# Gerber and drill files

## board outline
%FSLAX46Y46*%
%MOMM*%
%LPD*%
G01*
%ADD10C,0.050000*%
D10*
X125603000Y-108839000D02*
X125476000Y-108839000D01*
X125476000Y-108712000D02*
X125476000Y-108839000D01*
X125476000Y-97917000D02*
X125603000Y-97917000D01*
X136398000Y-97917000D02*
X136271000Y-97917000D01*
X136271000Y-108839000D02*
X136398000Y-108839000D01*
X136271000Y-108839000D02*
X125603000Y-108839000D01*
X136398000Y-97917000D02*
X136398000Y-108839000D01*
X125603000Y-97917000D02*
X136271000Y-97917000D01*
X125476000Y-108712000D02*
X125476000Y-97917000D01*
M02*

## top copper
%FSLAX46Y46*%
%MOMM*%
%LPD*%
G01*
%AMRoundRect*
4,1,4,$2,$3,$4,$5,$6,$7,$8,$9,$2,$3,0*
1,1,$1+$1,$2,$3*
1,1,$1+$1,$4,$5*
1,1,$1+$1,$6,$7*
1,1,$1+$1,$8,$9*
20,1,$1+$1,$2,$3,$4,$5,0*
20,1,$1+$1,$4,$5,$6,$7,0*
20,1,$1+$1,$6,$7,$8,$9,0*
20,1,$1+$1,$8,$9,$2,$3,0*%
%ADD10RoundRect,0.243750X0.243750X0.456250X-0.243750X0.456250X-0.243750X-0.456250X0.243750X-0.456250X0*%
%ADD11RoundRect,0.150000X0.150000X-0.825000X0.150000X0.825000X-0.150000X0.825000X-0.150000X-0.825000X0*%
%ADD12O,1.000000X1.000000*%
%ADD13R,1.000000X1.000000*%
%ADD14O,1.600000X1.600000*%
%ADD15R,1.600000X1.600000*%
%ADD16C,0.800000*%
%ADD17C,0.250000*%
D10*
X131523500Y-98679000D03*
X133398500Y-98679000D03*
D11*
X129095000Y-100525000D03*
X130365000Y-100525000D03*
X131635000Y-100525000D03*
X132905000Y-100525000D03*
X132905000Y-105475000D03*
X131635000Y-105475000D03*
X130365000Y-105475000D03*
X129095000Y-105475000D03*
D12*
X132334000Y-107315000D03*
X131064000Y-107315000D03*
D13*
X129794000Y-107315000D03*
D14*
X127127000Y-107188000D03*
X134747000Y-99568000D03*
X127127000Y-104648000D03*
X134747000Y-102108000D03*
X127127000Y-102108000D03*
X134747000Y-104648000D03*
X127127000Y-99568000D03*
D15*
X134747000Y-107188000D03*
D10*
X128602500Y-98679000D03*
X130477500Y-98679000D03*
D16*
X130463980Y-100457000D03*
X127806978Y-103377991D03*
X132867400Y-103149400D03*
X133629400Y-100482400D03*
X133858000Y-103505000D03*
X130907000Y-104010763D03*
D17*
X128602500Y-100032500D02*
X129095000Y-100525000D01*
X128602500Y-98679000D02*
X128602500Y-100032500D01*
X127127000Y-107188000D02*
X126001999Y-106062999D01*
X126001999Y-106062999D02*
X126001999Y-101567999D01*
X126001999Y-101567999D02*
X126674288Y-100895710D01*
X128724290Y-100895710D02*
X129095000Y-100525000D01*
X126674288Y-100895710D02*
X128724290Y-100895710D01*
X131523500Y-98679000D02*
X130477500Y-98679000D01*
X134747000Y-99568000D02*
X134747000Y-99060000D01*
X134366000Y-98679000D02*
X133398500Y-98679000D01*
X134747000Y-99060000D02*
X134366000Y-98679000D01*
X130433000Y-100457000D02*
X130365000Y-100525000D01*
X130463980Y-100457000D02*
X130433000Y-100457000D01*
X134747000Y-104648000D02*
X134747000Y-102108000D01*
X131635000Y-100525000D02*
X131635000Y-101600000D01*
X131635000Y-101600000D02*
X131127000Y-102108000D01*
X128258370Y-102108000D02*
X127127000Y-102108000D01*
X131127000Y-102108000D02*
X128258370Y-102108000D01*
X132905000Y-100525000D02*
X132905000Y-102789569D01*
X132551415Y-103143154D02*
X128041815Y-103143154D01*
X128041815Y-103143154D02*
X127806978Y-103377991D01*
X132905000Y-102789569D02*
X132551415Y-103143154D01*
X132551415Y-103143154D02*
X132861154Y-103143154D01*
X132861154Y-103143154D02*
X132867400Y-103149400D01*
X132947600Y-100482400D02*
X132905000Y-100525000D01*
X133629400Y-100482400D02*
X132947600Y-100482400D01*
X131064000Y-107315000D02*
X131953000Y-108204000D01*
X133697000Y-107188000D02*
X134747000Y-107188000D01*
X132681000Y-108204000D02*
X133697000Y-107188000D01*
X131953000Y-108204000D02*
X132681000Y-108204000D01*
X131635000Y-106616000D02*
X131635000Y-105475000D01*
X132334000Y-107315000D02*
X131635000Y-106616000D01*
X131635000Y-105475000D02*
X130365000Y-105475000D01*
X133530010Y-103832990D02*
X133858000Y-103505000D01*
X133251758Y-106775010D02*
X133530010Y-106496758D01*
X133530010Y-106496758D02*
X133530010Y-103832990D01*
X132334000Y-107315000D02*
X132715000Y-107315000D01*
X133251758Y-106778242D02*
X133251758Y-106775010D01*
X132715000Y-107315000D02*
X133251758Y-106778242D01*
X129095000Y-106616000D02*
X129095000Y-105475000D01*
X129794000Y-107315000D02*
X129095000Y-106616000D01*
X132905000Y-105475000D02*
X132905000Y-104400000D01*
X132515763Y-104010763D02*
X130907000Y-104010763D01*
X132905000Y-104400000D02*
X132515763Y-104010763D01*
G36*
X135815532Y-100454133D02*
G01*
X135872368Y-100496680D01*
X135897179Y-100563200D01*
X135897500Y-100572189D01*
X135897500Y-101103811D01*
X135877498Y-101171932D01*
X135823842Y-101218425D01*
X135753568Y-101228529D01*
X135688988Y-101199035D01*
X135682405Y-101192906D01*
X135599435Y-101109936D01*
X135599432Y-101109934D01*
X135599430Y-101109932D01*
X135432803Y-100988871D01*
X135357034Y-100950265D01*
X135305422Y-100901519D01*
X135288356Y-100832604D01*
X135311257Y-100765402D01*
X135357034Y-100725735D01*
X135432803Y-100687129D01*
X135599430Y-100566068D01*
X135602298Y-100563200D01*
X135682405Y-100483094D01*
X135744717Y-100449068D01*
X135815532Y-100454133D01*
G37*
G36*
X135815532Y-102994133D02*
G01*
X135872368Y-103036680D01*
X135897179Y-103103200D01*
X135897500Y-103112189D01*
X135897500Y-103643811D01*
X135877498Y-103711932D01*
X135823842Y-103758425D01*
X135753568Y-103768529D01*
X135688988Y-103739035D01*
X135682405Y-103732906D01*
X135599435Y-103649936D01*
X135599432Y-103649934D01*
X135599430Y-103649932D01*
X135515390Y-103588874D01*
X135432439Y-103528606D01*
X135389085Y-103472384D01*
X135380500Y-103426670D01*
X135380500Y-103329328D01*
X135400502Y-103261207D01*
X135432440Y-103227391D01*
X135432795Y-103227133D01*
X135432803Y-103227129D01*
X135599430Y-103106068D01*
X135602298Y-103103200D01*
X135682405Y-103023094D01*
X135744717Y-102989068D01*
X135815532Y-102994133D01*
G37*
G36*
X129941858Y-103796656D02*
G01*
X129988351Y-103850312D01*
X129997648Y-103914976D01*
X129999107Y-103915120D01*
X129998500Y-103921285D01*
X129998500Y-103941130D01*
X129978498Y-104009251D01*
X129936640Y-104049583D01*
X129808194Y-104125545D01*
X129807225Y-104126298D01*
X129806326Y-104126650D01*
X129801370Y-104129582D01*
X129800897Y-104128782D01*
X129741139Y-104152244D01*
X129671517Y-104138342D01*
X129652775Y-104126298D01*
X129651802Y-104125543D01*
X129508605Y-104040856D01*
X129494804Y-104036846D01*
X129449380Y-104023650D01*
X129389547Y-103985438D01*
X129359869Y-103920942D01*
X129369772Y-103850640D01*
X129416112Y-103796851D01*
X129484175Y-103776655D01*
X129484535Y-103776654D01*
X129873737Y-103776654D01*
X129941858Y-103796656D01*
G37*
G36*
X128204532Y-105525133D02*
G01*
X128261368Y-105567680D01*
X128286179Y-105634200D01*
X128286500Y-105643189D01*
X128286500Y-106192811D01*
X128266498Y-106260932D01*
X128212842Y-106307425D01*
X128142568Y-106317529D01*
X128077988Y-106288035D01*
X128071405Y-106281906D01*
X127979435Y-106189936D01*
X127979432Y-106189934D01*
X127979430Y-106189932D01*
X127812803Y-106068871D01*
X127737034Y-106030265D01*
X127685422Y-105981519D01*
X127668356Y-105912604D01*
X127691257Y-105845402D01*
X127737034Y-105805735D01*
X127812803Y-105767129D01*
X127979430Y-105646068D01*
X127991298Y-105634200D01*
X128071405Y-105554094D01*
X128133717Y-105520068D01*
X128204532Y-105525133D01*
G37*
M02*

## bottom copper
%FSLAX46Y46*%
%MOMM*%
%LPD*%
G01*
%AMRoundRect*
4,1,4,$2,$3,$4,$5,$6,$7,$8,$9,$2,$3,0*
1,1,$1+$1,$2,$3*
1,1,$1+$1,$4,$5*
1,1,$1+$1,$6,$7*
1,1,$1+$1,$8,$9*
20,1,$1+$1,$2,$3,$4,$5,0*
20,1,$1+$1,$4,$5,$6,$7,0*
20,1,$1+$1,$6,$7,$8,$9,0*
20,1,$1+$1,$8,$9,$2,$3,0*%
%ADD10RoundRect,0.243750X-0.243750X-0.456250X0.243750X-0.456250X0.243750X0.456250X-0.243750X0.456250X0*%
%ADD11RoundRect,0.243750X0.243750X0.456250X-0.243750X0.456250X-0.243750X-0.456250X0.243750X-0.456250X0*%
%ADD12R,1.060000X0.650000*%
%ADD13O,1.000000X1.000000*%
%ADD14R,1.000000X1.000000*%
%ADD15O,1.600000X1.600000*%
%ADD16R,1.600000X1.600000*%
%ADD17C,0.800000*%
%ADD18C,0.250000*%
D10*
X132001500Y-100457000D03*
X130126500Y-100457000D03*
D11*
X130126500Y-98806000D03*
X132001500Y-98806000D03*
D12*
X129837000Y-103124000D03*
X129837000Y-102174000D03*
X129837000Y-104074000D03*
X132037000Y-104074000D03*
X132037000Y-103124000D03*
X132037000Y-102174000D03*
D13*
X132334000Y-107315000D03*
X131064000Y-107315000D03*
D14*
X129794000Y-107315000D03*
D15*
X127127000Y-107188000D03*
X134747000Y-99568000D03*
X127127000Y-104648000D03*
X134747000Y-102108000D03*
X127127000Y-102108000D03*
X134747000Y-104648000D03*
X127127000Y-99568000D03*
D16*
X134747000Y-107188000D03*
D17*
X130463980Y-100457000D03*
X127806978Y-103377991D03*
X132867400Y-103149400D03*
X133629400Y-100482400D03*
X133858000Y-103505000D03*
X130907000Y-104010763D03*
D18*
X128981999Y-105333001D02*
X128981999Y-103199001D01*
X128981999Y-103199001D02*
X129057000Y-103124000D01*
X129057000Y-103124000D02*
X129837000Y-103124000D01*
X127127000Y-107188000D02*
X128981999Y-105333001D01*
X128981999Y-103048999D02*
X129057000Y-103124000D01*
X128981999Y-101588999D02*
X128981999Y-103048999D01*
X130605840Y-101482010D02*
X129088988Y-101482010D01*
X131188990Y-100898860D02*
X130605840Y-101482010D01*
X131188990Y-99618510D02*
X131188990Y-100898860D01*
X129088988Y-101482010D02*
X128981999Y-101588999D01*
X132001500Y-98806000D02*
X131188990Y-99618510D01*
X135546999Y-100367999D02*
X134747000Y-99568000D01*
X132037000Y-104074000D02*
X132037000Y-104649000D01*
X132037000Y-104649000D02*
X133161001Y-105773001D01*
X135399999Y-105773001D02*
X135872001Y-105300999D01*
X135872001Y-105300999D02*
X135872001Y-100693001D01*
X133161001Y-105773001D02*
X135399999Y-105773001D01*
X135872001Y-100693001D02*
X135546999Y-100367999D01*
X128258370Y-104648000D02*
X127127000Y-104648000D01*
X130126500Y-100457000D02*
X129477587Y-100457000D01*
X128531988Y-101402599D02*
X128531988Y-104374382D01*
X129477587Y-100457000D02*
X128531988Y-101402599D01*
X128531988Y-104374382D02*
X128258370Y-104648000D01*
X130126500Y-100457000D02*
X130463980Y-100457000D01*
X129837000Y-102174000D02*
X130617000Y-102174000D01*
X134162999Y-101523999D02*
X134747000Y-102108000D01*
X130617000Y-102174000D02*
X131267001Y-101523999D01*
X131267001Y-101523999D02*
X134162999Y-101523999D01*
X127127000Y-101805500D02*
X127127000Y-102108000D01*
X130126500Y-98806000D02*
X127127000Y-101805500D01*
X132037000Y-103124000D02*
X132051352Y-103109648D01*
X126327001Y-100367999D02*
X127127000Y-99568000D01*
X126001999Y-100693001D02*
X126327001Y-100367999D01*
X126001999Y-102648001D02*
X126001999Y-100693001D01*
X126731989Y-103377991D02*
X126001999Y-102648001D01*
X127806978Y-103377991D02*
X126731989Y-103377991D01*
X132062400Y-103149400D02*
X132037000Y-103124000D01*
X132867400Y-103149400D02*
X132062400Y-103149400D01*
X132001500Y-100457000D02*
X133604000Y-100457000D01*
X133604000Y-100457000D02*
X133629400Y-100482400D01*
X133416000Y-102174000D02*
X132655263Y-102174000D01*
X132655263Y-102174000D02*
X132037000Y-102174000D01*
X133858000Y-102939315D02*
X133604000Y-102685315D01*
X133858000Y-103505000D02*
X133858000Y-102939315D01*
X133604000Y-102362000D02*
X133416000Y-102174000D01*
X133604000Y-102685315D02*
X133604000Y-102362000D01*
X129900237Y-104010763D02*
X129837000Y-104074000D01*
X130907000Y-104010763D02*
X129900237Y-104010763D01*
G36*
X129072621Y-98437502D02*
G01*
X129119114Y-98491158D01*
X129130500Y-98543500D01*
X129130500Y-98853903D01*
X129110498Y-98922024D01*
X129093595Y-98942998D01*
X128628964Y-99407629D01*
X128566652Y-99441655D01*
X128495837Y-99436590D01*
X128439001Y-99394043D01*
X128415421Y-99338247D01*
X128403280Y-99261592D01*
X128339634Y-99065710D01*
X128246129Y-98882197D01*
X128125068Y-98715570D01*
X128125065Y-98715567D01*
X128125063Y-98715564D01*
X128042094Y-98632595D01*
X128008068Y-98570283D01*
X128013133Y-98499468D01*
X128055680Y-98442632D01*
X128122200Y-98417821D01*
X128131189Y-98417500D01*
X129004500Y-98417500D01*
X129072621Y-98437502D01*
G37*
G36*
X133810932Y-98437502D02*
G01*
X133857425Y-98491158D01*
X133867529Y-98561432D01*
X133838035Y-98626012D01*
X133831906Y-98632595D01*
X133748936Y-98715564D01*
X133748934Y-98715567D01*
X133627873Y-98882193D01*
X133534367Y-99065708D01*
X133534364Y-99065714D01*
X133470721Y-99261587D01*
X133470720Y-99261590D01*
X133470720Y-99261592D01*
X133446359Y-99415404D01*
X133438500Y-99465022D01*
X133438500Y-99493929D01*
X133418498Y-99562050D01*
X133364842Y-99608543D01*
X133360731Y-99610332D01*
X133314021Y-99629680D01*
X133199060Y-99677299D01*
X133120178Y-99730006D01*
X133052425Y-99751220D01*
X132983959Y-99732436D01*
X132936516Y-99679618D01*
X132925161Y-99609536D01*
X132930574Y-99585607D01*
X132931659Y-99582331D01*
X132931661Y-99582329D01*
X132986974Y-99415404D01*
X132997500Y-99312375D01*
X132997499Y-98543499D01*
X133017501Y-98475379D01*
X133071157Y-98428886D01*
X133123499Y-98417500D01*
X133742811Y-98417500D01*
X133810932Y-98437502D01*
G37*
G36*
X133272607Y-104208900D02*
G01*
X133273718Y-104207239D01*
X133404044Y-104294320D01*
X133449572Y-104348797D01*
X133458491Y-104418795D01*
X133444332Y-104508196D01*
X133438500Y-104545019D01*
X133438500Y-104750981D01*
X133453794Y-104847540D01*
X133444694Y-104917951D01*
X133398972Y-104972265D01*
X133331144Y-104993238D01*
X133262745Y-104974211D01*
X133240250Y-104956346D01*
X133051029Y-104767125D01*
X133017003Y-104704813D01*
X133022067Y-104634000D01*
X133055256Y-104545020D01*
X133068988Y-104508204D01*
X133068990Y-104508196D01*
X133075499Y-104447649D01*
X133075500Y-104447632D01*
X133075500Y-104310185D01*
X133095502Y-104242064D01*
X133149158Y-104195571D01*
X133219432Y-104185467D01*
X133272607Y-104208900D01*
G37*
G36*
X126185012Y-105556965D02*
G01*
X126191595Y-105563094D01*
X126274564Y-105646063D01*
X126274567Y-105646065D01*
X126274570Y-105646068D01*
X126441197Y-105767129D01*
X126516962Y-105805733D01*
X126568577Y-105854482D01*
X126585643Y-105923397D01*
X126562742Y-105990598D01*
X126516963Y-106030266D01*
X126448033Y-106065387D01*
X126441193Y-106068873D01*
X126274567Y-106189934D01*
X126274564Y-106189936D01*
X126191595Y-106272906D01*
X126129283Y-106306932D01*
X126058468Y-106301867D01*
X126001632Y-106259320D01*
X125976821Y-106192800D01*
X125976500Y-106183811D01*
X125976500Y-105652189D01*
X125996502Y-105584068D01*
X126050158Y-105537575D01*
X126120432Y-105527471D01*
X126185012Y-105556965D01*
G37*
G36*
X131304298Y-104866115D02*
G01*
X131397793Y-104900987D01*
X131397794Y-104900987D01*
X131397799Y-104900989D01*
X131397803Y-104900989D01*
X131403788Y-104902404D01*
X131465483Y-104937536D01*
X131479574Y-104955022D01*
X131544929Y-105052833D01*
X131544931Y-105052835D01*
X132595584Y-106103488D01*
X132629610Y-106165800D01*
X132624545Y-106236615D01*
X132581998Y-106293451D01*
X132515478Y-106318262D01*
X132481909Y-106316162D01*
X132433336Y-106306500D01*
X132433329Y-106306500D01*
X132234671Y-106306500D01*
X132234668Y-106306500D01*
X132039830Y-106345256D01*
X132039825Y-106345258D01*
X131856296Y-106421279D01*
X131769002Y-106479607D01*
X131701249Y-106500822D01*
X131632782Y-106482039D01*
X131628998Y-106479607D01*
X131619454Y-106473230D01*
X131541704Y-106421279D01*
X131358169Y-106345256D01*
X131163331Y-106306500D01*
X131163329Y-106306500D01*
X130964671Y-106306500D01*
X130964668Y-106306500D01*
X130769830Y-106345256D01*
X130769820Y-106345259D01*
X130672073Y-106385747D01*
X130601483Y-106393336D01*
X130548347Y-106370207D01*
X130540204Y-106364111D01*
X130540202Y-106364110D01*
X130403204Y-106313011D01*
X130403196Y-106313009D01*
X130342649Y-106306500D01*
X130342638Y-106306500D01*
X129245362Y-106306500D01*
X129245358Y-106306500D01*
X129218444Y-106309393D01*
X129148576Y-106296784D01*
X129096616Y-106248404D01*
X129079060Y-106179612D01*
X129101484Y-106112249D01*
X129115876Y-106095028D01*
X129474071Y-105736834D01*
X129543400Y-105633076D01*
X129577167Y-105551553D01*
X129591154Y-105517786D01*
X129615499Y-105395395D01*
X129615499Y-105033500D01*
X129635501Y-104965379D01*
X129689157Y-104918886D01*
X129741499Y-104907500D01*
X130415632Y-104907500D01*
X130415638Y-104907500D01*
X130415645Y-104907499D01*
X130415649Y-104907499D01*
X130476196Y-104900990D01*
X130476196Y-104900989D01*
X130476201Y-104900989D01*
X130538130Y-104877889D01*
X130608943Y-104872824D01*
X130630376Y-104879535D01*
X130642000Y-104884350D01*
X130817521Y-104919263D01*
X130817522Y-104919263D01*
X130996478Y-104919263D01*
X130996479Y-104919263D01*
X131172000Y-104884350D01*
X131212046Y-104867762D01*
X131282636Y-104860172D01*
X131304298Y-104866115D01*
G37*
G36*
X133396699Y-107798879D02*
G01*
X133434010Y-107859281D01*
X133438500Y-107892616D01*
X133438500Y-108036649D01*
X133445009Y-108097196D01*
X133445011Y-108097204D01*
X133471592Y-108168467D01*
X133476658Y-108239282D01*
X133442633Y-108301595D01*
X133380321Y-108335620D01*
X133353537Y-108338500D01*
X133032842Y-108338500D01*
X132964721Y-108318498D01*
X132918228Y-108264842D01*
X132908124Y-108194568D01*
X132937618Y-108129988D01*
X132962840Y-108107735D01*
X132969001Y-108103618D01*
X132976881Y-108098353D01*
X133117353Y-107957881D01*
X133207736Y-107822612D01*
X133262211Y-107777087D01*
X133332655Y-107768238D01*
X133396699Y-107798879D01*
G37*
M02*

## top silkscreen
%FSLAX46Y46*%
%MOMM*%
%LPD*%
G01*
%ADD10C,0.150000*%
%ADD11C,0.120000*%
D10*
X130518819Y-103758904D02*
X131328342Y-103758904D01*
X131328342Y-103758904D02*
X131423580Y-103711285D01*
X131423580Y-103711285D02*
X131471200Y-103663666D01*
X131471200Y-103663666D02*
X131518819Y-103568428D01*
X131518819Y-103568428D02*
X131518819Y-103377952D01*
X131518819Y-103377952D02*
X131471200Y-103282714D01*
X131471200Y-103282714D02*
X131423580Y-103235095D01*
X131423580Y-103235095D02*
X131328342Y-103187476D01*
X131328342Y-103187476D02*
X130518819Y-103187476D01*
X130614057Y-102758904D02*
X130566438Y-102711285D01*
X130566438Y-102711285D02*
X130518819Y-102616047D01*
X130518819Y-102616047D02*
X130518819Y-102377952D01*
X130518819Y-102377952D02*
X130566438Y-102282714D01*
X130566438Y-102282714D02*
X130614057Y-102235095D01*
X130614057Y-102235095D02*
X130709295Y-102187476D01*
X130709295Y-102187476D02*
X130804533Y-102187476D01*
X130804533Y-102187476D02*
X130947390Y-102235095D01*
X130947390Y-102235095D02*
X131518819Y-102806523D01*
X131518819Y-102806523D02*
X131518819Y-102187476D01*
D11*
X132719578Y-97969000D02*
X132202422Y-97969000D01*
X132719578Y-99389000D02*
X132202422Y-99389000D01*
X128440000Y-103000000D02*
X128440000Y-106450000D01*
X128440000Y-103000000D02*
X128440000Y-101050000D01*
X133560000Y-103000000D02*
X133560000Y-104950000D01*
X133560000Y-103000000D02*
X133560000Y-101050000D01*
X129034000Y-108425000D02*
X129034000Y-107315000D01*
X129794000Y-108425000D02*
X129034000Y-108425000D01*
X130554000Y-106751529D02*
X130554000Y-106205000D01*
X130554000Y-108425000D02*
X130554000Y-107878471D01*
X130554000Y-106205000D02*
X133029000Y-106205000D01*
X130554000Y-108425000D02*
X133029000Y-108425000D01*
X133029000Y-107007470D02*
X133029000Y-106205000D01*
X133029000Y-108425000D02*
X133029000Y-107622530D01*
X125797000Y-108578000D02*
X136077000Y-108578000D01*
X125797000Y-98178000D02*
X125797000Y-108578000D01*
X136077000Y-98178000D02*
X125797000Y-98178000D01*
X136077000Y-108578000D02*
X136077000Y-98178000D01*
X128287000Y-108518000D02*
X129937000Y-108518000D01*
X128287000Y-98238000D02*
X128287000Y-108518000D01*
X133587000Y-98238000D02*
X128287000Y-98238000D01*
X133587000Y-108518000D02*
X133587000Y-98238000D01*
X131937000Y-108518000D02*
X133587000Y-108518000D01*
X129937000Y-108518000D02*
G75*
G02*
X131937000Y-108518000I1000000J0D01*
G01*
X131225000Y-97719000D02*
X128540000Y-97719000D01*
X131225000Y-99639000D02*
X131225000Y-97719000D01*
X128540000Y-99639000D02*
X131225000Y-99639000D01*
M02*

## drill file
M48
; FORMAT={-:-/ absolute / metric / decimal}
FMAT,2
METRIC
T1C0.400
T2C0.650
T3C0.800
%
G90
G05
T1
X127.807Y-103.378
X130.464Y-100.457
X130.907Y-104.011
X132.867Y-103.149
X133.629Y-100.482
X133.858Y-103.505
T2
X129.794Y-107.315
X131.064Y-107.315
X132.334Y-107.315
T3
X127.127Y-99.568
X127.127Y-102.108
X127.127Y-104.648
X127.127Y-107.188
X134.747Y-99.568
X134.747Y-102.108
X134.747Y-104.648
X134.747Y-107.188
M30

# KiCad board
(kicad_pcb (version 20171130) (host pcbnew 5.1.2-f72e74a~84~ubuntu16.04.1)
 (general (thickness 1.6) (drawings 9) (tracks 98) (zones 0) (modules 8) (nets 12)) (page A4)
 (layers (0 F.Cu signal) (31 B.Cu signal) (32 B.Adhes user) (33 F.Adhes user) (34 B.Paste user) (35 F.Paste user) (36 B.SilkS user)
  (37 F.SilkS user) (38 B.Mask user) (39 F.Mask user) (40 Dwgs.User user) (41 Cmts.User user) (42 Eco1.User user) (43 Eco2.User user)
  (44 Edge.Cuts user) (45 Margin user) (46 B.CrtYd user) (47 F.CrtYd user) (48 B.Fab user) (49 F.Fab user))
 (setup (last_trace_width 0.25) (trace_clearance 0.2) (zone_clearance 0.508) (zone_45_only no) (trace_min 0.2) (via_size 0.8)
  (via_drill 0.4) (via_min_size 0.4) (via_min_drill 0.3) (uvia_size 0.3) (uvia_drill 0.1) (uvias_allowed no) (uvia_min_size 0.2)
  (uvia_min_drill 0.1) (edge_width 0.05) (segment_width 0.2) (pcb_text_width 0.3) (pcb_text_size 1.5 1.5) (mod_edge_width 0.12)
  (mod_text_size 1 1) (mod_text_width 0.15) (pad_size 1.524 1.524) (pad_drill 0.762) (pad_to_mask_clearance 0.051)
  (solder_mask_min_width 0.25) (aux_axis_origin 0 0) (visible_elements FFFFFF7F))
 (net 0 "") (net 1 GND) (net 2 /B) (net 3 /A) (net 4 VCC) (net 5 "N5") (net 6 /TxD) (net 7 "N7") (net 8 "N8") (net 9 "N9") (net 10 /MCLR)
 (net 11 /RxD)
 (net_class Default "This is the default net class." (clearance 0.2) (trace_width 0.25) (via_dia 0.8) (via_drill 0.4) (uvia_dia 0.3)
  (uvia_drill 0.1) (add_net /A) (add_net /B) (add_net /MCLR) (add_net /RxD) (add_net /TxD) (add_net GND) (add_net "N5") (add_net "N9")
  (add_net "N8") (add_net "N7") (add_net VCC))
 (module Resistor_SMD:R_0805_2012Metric (layer B.Cu) (at 131.064 100.457)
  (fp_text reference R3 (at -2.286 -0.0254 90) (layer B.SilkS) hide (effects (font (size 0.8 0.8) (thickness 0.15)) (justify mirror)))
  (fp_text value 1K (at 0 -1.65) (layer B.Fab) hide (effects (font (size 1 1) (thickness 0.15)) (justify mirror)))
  (pad 2 smd roundrect (at 0.9375 0) (size 0.975 1.4) (layers B.Cu B.Paste B.Mask) (roundrect_rratio 0.25) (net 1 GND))
  (pad 1 smd roundrect (at -0.9375 0) (size 0.975 1.4) (layers B.Cu B.Paste B.Mask) (roundrect_rratio 0.25) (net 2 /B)))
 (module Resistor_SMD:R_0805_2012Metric (layer B.Cu) (at 131.064 98.806 180)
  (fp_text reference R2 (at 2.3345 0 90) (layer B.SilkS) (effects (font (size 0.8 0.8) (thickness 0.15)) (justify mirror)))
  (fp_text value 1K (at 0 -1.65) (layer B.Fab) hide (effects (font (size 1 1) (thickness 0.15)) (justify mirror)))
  (pad 2 smd roundrect (at 0.9375 0 180) (size 0.975 1.4) (layers B.Cu B.Paste B.Mask) (roundrect_rratio 0.25) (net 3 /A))
  (pad 1 smd roundrect (at -0.9375 0 180) (size 0.975 1.4) (layers B.Cu B.Paste B.Mask) (roundrect_rratio 0.25) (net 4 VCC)))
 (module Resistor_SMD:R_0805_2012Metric (layer F.Cu) (at 132.461 98.679 180)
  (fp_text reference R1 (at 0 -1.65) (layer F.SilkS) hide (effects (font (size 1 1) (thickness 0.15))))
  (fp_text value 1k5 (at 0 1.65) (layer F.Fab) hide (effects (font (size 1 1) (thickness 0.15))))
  (fp_line (start -0.258578 0.71) (end 0.258578 0.71) (layer F.SilkS) (width 0.12))
  (fp_line (start -0.258578 -0.71) (end 0.258578 -0.71) (layer F.SilkS) (width 0.12))
  (pad 2 smd roundrect (at 0.9375 0 180) (size 0.975 1.4) (layers F.Cu F.Paste F.Mask) (roundrect_rratio 0.25) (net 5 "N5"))
  (pad 1 smd roundrect (at -0.9375 0 180) (size 0.975 1.4) (layers F.Cu F.Paste F.Mask) (roundrect_rratio 0.25) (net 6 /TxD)))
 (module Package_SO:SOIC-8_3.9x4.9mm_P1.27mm (layer F.Cu) (at 131 103 90)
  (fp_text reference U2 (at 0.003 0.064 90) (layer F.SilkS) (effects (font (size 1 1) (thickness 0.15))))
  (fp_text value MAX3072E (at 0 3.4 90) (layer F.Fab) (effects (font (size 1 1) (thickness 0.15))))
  (fp_line (start 0 -2.56) (end -3.45 -2.56) (layer F.SilkS) (width 0.12))
  (fp_line (start 0 -2.56) (end 1.95 -2.56) (layer F.SilkS) (width 0.12))
  (fp_line (start 0 2.56) (end -1.95 2.56) (layer F.SilkS) (width 0.12))
  (fp_line (start 0 2.56) (end 1.95 2.56) (layer F.SilkS) (width 0.12))
  (pad 8 smd roundrect (at 2.475 -1.905 90) (size 1.95 0.6) (layers F.Cu F.Paste F.Mask) (roundrect_rratio 0.25) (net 4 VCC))
  (pad 7 smd roundrect (at 2.475 -0.635 90) (size 1.95 0.6) (layers F.Cu F.Paste F.Mask) (roundrect_rratio 0.25) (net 2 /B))
  (pad 6 smd roundrect (at 2.475 0.635 90) (size 1.95 0.6) (layers F.Cu F.Paste F.Mask) (roundrect_rratio 0.25) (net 3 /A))
  (pad 5 smd roundrect (at 2.475 1.905 90) (size 1.95 0.6) (layers F.Cu F.Paste F.Mask) (roundrect_rratio 0.25) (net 1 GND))
  (pad 4 smd roundrect (at -2.475 1.905 90) (size 1.95 0.6) (layers F.Cu F.Paste F.Mask) (roundrect_rratio 0.25) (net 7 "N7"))
  (pad 3 smd roundrect (at -2.475 0.635 90) (size 1.95 0.6) (layers F.Cu F.Paste F.Mask) (roundrect_rratio 0.25) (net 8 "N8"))
  (pad 2 smd roundrect (at -2.475 -0.635 90) (size 1.95 0.6) (layers F.Cu F.Paste F.Mask) (roundrect_rratio 0.25) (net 8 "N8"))
  (pad 1 smd roundrect (at -2.475 -1.905 90) (size 1.95 0.6) (layers F.Cu F.Paste F.Mask) (roundrect_rratio 0.25) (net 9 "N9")))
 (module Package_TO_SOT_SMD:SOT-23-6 (layer B.Cu) (at 130.937 103.124 180)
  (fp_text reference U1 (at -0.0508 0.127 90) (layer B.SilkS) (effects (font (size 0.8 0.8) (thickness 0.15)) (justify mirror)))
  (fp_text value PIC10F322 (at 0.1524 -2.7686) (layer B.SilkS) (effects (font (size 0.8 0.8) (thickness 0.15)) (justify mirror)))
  (pad 5 smd rect (at 1.1 0 180) (size 1.06 0.65) (layers B.Cu B.Paste B.Mask) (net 4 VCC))
  (pad 6 smd rect (at 1.1 0.95 180) (size 1.06 0.65) (layers B.Cu B.Paste B.Mask) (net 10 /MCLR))
  (pad 4 smd rect (at 1.1 -0.95 180) (size 1.06 0.65) (layers B.Cu B.Paste B.Mask) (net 7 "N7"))
  (pad 3 smd rect (at -1.1 -0.95 180) (size 1.06 0.65) (layers B.Cu B.Paste B.Mask) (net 6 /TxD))
  (pad 2 smd rect (at -1.1 0 180) (size 1.06 0.65) (layers B.Cu B.Paste B.Mask) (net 1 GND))
  (pad 1 smd rect (at -1.1 0.95 180) (size 1.06 0.65) (layers B.Cu B.Paste B.Mask) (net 8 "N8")))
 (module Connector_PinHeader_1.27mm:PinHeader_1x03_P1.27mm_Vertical (layer F.Cu) (at 129.794 107.315 90)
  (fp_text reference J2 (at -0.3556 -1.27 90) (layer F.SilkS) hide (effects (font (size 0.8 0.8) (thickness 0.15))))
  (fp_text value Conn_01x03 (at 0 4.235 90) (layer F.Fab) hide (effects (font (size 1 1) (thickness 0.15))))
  (fp_line (start -1.11 -0.76) (end 0 -0.76) (layer F.SilkS) (width 0.12))
  (fp_line (start -1.11 0) (end -1.11 -0.76) (layer F.SilkS) (width 0.12))
  (fp_line (start 0.563471 0.76) (end 1.11 0.76) (layer F.SilkS) (width 0.12))
  (fp_line (start -1.11 0.76) (end -0.563471 0.76) (layer F.SilkS) (width 0.12))
  (fp_line (start 1.11 0.76) (end 1.11 3.235) (layer F.SilkS) (width 0.12))
  (fp_line (start -1.11 0.76) (end -1.11 3.235) (layer F.SilkS) (width 0.12))
  (fp_line (start 0.30753 3.235) (end 1.11 3.235) (layer F.SilkS) (width 0.12))
  (fp_line (start -1.11 3.235) (end -0.30753 3.235) (layer F.SilkS) (width 0.12))
  (pad 3 thru_hole oval (at 0 2.54 90) (size 1 1) (drill 0.65) (layers *.Cu *.Mask) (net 8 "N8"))
  (pad 2 thru_hole oval (at 0 1.27 90) (size 1 1) (drill 0.65) (layers *.Cu *.Mask) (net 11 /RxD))
  (pad 1 thru_hole rect (at 0 0 90) (size 1 1) (drill 0.65) (layers *.Cu *.Mask) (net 9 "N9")))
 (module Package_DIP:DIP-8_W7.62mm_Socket (layer F.Cu) (at 134.747 107.188 180)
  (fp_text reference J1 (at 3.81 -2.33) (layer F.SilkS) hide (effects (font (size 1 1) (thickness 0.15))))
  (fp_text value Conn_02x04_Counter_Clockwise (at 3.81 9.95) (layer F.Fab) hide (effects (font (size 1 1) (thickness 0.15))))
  (fp_line (start 8.95 -1.39) (end -1.33 -1.39) (layer F.SilkS) (width 0.12))
  (fp_line (start 8.95 9.01) (end 8.95 -1.39) (layer F.SilkS) (width 0.12))
  (fp_line (start -1.33 9.01) (end 8.95 9.01) (layer F.SilkS) (width 0.12))
  (fp_line (start -1.33 -1.39) (end -1.33 9.01) (layer F.SilkS) (width 0.12))
  (fp_line (start 6.46 -1.33) (end 4.81 -1.33) (layer F.SilkS) (width 0.12))
  (fp_line (start 6.46 8.95) (end 6.46 -1.33) (layer F.SilkS) (width 0.12))
  (fp_line (start 1.16 8.95) (end 6.46 8.95) (layer F.SilkS) (width 0.12))
  (fp_line (start 1.16 -1.33) (end 1.16 8.95) (layer F.SilkS) (width 0.12))
  (fp_line (start 2.81 -1.33) (end 1.16 -1.33) (layer F.SilkS) (width 0.12))
  (fp_arc (start 3.81 -1.33) (end 2.81 -1.33) (angle -180) (layer F.SilkS) (width 0.12))
  (pad 8 thru_hole oval (at 7.62 0 180) (size 1.6 1.6) (drill 0.8) (layers *.Cu *.Mask) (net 4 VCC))
  (pad 4 thru_hole oval (at 0 7.62 180) (size 1.6 1.6) (drill 0.8) (layers *.Cu *.Mask) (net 6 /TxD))
  (pad 7 thru_hole oval (at 7.62 2.54 180) (size 1.6 1.6) (drill 0.8) (layers *.Cu *.Mask) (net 2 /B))
  (pad 3 thru_hole oval (at 0 5.08 180) (size 1.6 1.6) (drill 0.8) (layers *.Cu *.Mask) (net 10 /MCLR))
  (pad 6 thru_hole oval (at 7.62 5.08 180) (size 1.6 1.6) (drill 0.8) (layers *.Cu *.Mask) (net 3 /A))
  (pad 2 thru_hole oval (at 0 2.54 180) (size 1.6 1.6) (drill 0.8) (layers *.Cu *.Mask) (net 10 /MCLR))
  (pad 5 thru_hole oval (at 7.62 7.62 180) (size 1.6 1.6) (drill 0.8) (layers *.Cu *.Mask) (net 1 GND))
  (pad 1 thru_hole rect (at 0 0 180) (size 1.6 1.6) (drill 0.8) (layers *.Cu *.Mask) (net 11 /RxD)))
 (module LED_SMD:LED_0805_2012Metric (layer F.Cu) (at 129.54 98.679 180)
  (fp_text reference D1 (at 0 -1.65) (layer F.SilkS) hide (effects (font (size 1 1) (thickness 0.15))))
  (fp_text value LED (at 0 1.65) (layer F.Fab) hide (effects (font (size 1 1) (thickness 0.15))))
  (fp_line (start -1.685 0.96) (end 1 0.96) (layer F.SilkS) (width 0.12))
  (fp_line (start -1.685 -0.96) (end -1.685 0.96) (layer F.SilkS) (width 0.12))
  (fp_line (start 1 -0.96) (end -1.685 -0.96) (layer F.SilkS) (width 0.12))
  (pad 2 smd roundrect (at 0.9375 0 180) (size 0.975 1.4) (layers F.Cu F.Paste F.Mask) (roundrect_rratio 0.25) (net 4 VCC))
  (pad 1 smd roundrect (at -0.9375 0 180) (size 0.975 1.4) (layers F.Cu F.Paste F.Mask) (roundrect_rratio 0.25) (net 5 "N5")))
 (gr_line (start 125.603 108.839) (end 125.476 108.839) (layer Edge.Cuts) (width 0.05))
 (gr_line (start 125.476 108.712) (end 125.476 108.839) (layer Edge.Cuts) (width 0.05))
 (gr_line (start 125.476 97.917) (end 125.603 97.917) (layer Edge.Cuts) (width 0.05))
 (gr_line (start 136.398 97.917) (end 136.271 97.917) (layer Edge.Cuts) (width 0.05))
 (gr_line (start 136.271 108.839) (end 136.398 108.839) (layer Edge.Cuts) (width 0.05))
 (gr_line (start 136.271 108.839) (end 125.603 108.839) (layer Edge.Cuts) (width 0.05))
 (gr_line (start 136.398 97.917) (end 136.398 108.839) (layer Edge.Cuts) (width 0.05))
 (gr_line (start 125.603 97.917) (end 136.271 97.917) (layer Edge.Cuts) (width 0.05))
 (gr_line (start 125.476 108.712) (end 125.476 97.917) (layer Edge.Cuts) (width 0.05))
 (segment (start 128.6025 100.0325) (end 129.095 100.525) (width 0.25) (layer F.Cu) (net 4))
 (segment (start 128.6025 98.679) (end 128.6025 100.0325) (width 0.25) (layer F.Cu) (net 4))
 (segment (start 127.127 107.188) (end 126.001999 106.062999) (width 0.25) (layer F.Cu) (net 4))
 (segment (start 126.001999 106.062999) (end 126.001999 101.567999) (width 0.25) (layer F.Cu) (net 4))
 (segment (start 126.001999 101.567999) (end 126.674288 100.89571) (width 0.25) (layer F.Cu) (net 4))
 (segment (start 128.72429 100.89571) (end 129.095 100.525) (width 0.25) (layer F.Cu) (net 4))
 (segment (start 126.674288 100.89571) (end 128.72429 100.89571) (width 0.25) (layer F.Cu) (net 4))
 (segment (start 128.981999 105.333001) (end 128.981999 103.199001) (width 0.25) (layer B.Cu) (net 4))
 (segment (start 128.981999 103.199001) (end 129.057 103.124) (width 0.25) (layer B.Cu) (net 4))
 (segment (start 129.057 103.124) (end 129.837 103.124) (width 0.25) (layer B.Cu) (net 4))
 (segment (start 127.127 107.188) (end 128.981999 105.333001) (width 0.25) (layer B.Cu) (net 4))
 (segment (start 128.981999 103.048999) (end 129.057 103.124) (width 0.25) (layer B.Cu) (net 4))
 (segment (start 128.981999 101.588999) (end 128.981999 103.048999) (width 0.25) (layer B.Cu) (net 4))
 (segment (start 130.60584 101.48201) (end 129.088988 101.48201) (width 0.25) (layer B.Cu) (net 4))
 (segment (start 131.18899 100.89886) (end 130.60584 101.48201) (width 0.25) (layer B.Cu) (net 4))
 (segment (start 131.18899 99.61851) (end 131.18899 100.89886) (width 0.25) (layer B.Cu) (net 4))
 (segment (start 129.088988 101.48201) (end 128.981999 101.588999) (width 0.25) (layer B.Cu) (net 4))
 (segment (start 132.0015 98.806) (end 131.18899 99.61851) (width 0.25) (layer B.Cu) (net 4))
 (segment (start 131.5235 98.679) (end 130.4775 98.679) (width 0.25) (layer F.Cu) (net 5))
 (segment (start 135.546999 100.367999) (end 134.747 99.568) (width 0.25) (layer B.Cu) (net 6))
 (segment (start 132.037 104.074) (end 132.037 104.649) (width 0.25) (layer B.Cu) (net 6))
 (segment (start 132.037 104.649) (end 133.161001 105.773001) (width 0.25) (layer B.Cu) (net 6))
 (segment (start 135.399999 105.773001) (end 135.872001 105.300999) (width 0.25) (layer B.Cu) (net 6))
 (segment (start 135.872001 105.300999) (end 135.872001 100.693001) (width 0.25) (layer B.Cu) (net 6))
 (segment (start 133.161001 105.773001) (end 135.399999 105.773001) (width 0.25) (layer B.Cu) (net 6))
 (segment (start 135.872001 100.693001) (end 135.546999 100.367999) (width 0.25) (layer B.Cu) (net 6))
 (segment (start 134.747 99.568) (end 134.747 99.06) (width 0.25) (layer F.Cu) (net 6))
 (segment (start 134.366 98.679) (end 133.3985 98.679) (width 0.25) (layer F.Cu) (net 6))
 (segment (start 134.747 99.06) (end 134.366 98.679) (width 0.25) (layer F.Cu) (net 6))
 (segment (start 128.25837 104.648) (end 127.127 104.648) (width 0.25) (layer B.Cu) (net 2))
 (segment (start 130.1265 100.457) (end 129.477587 100.457) (width 0.25) (layer B.Cu) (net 2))
 (segment (start 128.531988 101.402599) (end 128.531988 104.374382) (width 0.25) (layer B.Cu) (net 2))
 (segment (start 129.477587 100.457) (end 128.531988 101.402599) (width 0.25) (layer B.Cu) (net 2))
 (segment (start 128.531988 104.374382) (end 128.25837 104.648) (width 0.25) (layer B.Cu) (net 2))
 (segment (start 130.1265 100.457) (end 130.46398 100.457) (width 0.25) (layer B.Cu) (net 2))
 (via (at 130.46398 100.457) (size 0.8) (drill 0.4) (layers F.Cu B.Cu) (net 2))
 (segment (start 130.433 100.457) (end 130.365 100.525) (width 0.25) (layer F.Cu) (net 2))
 (segment (start 130.46398 100.457) (end 130.433 100.457) (width 0.25) (layer F.Cu) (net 2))
 (segment (start 129.837 102.174) (end 130.617 102.174) (width 0.25) (layer B.Cu) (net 10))
 (segment (start 134.162999 101.523999) (end 134.747 102.108) (width 0.25) (layer B.Cu) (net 10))
 (segment (start 130.617 102.174) (end 131.267001 101.523999) (width 0.25) (layer B.Cu) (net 10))
 (segment (start 131.267001 101.523999) (end 134.162999 101.523999) (width 0.25) (layer B.Cu) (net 10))
 (segment (start 134.747 104.648) (end 134.747 102.108) (width 0.25) (layer F.Cu) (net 10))
 (segment (start 127.127 101.8055) (end 127.127 102.108) (width 0.25) (layer B.Cu) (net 3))
 (segment (start 130.1265 98.806) (end 127.127 101.8055) (width 0.25) (layer B.Cu) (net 3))
 (segment (start 131.635 100.525) (end 131.635 101.6) (width 0.25) (layer F.Cu) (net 3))
 (segment (start 131.635 101.6) (end 131.127 102.108) (width 0.25) (layer F.Cu) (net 3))
 (segment (start 128.25837 102.108) (end 127.127 102.108) (width 0.25) (layer F.Cu) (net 3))
 (segment (start 131.127 102.108) (end 128.25837 102.108) (width 0.25) (layer F.Cu) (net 3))
 (segment (start 132.037 103.124) (end 132.051352 103.109648) (width 0.25) (layer B.Cu) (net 1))
 (segment (start 132.905 100.525) (end 132.905 102.789569) (width 0.25) (layer F.Cu) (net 1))
 (via (at 127.806978 103.377991) (size 0.8) (drill 0.4) (layers F.Cu B.Cu) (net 1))
 (segment (start 132.551415 103.143154) (end 128.041815 103.143154) (width 0.25) (layer F.Cu) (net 1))
 (segment (start 128.041815 103.143154) (end 127.806978 103.377991) (width 0.25) (layer F.Cu) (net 1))
 (segment (start 126.327001 100.367999) (end 127.127 99.568) (width 0.25) (layer B.Cu) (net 1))
 (segment (start 126.001999 100.693001) (end 126.327001 100.367999) (width 0.25) (layer B.Cu) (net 1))
 (segment (start 126.001999 102.648001) (end 126.001999 100.693001) (width 0.25) (layer B.Cu) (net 1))
 (segment (start 126.731989 103.377991) (end 126.001999 102.648001) (width 0.25) (layer B.Cu) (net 1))
 (segment (start 127.806978 103.377991) (end 126.731989 103.377991) (width 0.25) (layer B.Cu) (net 1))
 (segment (start 132.905 102.789569) (end 132.551415 103.143154) (width 0.25) (layer F.Cu) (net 1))
 (segment (start 132.551415 103.143154) (end 132.861154 103.143154) (width 0.25) (layer F.Cu) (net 1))
 (via (at 132.8674 103.1494) (size 0.8) (drill 0.4) (layers F.Cu B.Cu) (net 1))
 (segment (start 132.861154 103.143154) (end 132.8674 103.1494) (width 0.25) (layer F.Cu) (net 1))
 (segment (start 132.0624 103.1494) (end 132.037 103.124) (width 0.25) (layer B.Cu) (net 1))
 (segment (start 132.8674 103.1494) (end 132.0624 103.1494) (width 0.25) (layer B.Cu) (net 1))
 (via (at 133.6294 100.4824) (size 0.8) (drill 0.4) (layers F.Cu B.Cu) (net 1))
 (segment (start 132.0015 100.457) (end 133.604 100.457) (width 0.25) (layer B.Cu) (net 1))
 (segment (start 133.604 100.457) (end 133.6294 100.4824) (width 0.25) (layer B.Cu) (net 1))
 (segment (start 132.9476 100.4824) (end 132.905 100.525) (width 0.25) (layer F.Cu) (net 1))
 (segment (start 133.6294 100.4824) (end 132.9476 100.4824) (width 0.25) (layer F.Cu) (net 1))
 (segment (start 131.064 107.315) (end 131.953 108.204) (width 0.25) (layer F.Cu) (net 11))
 (segment (start 133.697 107.188) (end 134.747 107.188) (width 0.25) (layer F.Cu) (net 11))
 (segment (start 132.681 108.204) (end 133.697 107.188) (width 0.25) (layer F.Cu) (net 11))
 (segment (start 131.953 108.204) (end 132.681 108.204) (width 0.25) (layer F.Cu) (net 11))
 (segment (start 131.635 106.616) (end 131.635 105.475) (width 0.25) (layer F.Cu) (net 8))
 (segment (start 132.334 107.315) (end 131.635 106.616) (width 0.25) (layer F.Cu) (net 8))
 (segment (start 131.635 105.475) (end 130.365 105.475) (width 0.25) (layer F.Cu) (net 8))
 (segment (start 133.53001 103.83299) (end 133.858 103.505) (width 0.25) (layer F.Cu) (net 8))
 (segment (start 133.251758 106.77501) (end 133.53001 106.496758) (width 0.25) (layer F.Cu) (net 8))
 (via (at 133.858 103.505) (size 0.8) (drill 0.4) (layers F.Cu B.Cu) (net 8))
 (segment (start 133.53001 106.496758) (end 133.53001 103.83299) (width 0.25) (layer F.Cu) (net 8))
 (segment (start 132.334 107.315) (end 132.715 107.315) (width 0.25) (layer F.Cu) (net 8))
 (segment (start 133.251758 106.778242) (end 133.251758 106.77501) (width 0.25) (layer F.Cu) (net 8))
 (segment (start 132.715 107.315) (end 133.251758 106.778242) (width 0.25) (layer F.Cu) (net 8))
 (segment (start 133.416 102.174) (end 132.655263 102.174) (width 0.25) (layer B.Cu) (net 8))
 (segment (start 132.655263 102.174) (end 132.037 102.174) (width 0.25) (layer B.Cu) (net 8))
 (segment (start 133.858 102.939315) (end 133.604 102.685315) (width 0.25) (layer B.Cu) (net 8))
 (segment (start 133.858 103.505) (end 133.858 102.939315) (width 0.25) (layer B.Cu) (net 8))
 (segment (start 133.604 102.362) (end 133.416 102.174) (width 0.25) (layer B.Cu) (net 8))
 (segment (start 133.604 102.685315) (end 133.604 102.362) (width 0.25) (layer B.Cu) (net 8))
 (segment (start 129.095 106.616) (end 129.095 105.475) (width 0.25) (layer F.Cu) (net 9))
 (segment (start 129.794 107.315) (end 129.095 106.616) (width 0.25) (layer F.Cu) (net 9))
 (via (at 130.907 104.010763) (size 0.8) (drill 0.4) (layers F.Cu B.Cu) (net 7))
 (segment (start 132.905 105.475) (end 132.905 104.4) (width 0.25) (layer F.Cu) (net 7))
 (segment (start 132.515763 104.010763) (end 130.907 104.010763) (width 0.25) (layer F.Cu) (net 7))
 (segment (start 132.905 104.4) (end 132.515763 104.010763) (width 0.25) (layer F.Cu) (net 7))
 (segment (start 129.900237 104.010763) (end 129.837 104.074) (width 0.25) (layer B.Cu) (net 7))
 (segment (start 130.907 104.010763) (end 129.900237 104.010763) (width 0.25) (layer B.Cu) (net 7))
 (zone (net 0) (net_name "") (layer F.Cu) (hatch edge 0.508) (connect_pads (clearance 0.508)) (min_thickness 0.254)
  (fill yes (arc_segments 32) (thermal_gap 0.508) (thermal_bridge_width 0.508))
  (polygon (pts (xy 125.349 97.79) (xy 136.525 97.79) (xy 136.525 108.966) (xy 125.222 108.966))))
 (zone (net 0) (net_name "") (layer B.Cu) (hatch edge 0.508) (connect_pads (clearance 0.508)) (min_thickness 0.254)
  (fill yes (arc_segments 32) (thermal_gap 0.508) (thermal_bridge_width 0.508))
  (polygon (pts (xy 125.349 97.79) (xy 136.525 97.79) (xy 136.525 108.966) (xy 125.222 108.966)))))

